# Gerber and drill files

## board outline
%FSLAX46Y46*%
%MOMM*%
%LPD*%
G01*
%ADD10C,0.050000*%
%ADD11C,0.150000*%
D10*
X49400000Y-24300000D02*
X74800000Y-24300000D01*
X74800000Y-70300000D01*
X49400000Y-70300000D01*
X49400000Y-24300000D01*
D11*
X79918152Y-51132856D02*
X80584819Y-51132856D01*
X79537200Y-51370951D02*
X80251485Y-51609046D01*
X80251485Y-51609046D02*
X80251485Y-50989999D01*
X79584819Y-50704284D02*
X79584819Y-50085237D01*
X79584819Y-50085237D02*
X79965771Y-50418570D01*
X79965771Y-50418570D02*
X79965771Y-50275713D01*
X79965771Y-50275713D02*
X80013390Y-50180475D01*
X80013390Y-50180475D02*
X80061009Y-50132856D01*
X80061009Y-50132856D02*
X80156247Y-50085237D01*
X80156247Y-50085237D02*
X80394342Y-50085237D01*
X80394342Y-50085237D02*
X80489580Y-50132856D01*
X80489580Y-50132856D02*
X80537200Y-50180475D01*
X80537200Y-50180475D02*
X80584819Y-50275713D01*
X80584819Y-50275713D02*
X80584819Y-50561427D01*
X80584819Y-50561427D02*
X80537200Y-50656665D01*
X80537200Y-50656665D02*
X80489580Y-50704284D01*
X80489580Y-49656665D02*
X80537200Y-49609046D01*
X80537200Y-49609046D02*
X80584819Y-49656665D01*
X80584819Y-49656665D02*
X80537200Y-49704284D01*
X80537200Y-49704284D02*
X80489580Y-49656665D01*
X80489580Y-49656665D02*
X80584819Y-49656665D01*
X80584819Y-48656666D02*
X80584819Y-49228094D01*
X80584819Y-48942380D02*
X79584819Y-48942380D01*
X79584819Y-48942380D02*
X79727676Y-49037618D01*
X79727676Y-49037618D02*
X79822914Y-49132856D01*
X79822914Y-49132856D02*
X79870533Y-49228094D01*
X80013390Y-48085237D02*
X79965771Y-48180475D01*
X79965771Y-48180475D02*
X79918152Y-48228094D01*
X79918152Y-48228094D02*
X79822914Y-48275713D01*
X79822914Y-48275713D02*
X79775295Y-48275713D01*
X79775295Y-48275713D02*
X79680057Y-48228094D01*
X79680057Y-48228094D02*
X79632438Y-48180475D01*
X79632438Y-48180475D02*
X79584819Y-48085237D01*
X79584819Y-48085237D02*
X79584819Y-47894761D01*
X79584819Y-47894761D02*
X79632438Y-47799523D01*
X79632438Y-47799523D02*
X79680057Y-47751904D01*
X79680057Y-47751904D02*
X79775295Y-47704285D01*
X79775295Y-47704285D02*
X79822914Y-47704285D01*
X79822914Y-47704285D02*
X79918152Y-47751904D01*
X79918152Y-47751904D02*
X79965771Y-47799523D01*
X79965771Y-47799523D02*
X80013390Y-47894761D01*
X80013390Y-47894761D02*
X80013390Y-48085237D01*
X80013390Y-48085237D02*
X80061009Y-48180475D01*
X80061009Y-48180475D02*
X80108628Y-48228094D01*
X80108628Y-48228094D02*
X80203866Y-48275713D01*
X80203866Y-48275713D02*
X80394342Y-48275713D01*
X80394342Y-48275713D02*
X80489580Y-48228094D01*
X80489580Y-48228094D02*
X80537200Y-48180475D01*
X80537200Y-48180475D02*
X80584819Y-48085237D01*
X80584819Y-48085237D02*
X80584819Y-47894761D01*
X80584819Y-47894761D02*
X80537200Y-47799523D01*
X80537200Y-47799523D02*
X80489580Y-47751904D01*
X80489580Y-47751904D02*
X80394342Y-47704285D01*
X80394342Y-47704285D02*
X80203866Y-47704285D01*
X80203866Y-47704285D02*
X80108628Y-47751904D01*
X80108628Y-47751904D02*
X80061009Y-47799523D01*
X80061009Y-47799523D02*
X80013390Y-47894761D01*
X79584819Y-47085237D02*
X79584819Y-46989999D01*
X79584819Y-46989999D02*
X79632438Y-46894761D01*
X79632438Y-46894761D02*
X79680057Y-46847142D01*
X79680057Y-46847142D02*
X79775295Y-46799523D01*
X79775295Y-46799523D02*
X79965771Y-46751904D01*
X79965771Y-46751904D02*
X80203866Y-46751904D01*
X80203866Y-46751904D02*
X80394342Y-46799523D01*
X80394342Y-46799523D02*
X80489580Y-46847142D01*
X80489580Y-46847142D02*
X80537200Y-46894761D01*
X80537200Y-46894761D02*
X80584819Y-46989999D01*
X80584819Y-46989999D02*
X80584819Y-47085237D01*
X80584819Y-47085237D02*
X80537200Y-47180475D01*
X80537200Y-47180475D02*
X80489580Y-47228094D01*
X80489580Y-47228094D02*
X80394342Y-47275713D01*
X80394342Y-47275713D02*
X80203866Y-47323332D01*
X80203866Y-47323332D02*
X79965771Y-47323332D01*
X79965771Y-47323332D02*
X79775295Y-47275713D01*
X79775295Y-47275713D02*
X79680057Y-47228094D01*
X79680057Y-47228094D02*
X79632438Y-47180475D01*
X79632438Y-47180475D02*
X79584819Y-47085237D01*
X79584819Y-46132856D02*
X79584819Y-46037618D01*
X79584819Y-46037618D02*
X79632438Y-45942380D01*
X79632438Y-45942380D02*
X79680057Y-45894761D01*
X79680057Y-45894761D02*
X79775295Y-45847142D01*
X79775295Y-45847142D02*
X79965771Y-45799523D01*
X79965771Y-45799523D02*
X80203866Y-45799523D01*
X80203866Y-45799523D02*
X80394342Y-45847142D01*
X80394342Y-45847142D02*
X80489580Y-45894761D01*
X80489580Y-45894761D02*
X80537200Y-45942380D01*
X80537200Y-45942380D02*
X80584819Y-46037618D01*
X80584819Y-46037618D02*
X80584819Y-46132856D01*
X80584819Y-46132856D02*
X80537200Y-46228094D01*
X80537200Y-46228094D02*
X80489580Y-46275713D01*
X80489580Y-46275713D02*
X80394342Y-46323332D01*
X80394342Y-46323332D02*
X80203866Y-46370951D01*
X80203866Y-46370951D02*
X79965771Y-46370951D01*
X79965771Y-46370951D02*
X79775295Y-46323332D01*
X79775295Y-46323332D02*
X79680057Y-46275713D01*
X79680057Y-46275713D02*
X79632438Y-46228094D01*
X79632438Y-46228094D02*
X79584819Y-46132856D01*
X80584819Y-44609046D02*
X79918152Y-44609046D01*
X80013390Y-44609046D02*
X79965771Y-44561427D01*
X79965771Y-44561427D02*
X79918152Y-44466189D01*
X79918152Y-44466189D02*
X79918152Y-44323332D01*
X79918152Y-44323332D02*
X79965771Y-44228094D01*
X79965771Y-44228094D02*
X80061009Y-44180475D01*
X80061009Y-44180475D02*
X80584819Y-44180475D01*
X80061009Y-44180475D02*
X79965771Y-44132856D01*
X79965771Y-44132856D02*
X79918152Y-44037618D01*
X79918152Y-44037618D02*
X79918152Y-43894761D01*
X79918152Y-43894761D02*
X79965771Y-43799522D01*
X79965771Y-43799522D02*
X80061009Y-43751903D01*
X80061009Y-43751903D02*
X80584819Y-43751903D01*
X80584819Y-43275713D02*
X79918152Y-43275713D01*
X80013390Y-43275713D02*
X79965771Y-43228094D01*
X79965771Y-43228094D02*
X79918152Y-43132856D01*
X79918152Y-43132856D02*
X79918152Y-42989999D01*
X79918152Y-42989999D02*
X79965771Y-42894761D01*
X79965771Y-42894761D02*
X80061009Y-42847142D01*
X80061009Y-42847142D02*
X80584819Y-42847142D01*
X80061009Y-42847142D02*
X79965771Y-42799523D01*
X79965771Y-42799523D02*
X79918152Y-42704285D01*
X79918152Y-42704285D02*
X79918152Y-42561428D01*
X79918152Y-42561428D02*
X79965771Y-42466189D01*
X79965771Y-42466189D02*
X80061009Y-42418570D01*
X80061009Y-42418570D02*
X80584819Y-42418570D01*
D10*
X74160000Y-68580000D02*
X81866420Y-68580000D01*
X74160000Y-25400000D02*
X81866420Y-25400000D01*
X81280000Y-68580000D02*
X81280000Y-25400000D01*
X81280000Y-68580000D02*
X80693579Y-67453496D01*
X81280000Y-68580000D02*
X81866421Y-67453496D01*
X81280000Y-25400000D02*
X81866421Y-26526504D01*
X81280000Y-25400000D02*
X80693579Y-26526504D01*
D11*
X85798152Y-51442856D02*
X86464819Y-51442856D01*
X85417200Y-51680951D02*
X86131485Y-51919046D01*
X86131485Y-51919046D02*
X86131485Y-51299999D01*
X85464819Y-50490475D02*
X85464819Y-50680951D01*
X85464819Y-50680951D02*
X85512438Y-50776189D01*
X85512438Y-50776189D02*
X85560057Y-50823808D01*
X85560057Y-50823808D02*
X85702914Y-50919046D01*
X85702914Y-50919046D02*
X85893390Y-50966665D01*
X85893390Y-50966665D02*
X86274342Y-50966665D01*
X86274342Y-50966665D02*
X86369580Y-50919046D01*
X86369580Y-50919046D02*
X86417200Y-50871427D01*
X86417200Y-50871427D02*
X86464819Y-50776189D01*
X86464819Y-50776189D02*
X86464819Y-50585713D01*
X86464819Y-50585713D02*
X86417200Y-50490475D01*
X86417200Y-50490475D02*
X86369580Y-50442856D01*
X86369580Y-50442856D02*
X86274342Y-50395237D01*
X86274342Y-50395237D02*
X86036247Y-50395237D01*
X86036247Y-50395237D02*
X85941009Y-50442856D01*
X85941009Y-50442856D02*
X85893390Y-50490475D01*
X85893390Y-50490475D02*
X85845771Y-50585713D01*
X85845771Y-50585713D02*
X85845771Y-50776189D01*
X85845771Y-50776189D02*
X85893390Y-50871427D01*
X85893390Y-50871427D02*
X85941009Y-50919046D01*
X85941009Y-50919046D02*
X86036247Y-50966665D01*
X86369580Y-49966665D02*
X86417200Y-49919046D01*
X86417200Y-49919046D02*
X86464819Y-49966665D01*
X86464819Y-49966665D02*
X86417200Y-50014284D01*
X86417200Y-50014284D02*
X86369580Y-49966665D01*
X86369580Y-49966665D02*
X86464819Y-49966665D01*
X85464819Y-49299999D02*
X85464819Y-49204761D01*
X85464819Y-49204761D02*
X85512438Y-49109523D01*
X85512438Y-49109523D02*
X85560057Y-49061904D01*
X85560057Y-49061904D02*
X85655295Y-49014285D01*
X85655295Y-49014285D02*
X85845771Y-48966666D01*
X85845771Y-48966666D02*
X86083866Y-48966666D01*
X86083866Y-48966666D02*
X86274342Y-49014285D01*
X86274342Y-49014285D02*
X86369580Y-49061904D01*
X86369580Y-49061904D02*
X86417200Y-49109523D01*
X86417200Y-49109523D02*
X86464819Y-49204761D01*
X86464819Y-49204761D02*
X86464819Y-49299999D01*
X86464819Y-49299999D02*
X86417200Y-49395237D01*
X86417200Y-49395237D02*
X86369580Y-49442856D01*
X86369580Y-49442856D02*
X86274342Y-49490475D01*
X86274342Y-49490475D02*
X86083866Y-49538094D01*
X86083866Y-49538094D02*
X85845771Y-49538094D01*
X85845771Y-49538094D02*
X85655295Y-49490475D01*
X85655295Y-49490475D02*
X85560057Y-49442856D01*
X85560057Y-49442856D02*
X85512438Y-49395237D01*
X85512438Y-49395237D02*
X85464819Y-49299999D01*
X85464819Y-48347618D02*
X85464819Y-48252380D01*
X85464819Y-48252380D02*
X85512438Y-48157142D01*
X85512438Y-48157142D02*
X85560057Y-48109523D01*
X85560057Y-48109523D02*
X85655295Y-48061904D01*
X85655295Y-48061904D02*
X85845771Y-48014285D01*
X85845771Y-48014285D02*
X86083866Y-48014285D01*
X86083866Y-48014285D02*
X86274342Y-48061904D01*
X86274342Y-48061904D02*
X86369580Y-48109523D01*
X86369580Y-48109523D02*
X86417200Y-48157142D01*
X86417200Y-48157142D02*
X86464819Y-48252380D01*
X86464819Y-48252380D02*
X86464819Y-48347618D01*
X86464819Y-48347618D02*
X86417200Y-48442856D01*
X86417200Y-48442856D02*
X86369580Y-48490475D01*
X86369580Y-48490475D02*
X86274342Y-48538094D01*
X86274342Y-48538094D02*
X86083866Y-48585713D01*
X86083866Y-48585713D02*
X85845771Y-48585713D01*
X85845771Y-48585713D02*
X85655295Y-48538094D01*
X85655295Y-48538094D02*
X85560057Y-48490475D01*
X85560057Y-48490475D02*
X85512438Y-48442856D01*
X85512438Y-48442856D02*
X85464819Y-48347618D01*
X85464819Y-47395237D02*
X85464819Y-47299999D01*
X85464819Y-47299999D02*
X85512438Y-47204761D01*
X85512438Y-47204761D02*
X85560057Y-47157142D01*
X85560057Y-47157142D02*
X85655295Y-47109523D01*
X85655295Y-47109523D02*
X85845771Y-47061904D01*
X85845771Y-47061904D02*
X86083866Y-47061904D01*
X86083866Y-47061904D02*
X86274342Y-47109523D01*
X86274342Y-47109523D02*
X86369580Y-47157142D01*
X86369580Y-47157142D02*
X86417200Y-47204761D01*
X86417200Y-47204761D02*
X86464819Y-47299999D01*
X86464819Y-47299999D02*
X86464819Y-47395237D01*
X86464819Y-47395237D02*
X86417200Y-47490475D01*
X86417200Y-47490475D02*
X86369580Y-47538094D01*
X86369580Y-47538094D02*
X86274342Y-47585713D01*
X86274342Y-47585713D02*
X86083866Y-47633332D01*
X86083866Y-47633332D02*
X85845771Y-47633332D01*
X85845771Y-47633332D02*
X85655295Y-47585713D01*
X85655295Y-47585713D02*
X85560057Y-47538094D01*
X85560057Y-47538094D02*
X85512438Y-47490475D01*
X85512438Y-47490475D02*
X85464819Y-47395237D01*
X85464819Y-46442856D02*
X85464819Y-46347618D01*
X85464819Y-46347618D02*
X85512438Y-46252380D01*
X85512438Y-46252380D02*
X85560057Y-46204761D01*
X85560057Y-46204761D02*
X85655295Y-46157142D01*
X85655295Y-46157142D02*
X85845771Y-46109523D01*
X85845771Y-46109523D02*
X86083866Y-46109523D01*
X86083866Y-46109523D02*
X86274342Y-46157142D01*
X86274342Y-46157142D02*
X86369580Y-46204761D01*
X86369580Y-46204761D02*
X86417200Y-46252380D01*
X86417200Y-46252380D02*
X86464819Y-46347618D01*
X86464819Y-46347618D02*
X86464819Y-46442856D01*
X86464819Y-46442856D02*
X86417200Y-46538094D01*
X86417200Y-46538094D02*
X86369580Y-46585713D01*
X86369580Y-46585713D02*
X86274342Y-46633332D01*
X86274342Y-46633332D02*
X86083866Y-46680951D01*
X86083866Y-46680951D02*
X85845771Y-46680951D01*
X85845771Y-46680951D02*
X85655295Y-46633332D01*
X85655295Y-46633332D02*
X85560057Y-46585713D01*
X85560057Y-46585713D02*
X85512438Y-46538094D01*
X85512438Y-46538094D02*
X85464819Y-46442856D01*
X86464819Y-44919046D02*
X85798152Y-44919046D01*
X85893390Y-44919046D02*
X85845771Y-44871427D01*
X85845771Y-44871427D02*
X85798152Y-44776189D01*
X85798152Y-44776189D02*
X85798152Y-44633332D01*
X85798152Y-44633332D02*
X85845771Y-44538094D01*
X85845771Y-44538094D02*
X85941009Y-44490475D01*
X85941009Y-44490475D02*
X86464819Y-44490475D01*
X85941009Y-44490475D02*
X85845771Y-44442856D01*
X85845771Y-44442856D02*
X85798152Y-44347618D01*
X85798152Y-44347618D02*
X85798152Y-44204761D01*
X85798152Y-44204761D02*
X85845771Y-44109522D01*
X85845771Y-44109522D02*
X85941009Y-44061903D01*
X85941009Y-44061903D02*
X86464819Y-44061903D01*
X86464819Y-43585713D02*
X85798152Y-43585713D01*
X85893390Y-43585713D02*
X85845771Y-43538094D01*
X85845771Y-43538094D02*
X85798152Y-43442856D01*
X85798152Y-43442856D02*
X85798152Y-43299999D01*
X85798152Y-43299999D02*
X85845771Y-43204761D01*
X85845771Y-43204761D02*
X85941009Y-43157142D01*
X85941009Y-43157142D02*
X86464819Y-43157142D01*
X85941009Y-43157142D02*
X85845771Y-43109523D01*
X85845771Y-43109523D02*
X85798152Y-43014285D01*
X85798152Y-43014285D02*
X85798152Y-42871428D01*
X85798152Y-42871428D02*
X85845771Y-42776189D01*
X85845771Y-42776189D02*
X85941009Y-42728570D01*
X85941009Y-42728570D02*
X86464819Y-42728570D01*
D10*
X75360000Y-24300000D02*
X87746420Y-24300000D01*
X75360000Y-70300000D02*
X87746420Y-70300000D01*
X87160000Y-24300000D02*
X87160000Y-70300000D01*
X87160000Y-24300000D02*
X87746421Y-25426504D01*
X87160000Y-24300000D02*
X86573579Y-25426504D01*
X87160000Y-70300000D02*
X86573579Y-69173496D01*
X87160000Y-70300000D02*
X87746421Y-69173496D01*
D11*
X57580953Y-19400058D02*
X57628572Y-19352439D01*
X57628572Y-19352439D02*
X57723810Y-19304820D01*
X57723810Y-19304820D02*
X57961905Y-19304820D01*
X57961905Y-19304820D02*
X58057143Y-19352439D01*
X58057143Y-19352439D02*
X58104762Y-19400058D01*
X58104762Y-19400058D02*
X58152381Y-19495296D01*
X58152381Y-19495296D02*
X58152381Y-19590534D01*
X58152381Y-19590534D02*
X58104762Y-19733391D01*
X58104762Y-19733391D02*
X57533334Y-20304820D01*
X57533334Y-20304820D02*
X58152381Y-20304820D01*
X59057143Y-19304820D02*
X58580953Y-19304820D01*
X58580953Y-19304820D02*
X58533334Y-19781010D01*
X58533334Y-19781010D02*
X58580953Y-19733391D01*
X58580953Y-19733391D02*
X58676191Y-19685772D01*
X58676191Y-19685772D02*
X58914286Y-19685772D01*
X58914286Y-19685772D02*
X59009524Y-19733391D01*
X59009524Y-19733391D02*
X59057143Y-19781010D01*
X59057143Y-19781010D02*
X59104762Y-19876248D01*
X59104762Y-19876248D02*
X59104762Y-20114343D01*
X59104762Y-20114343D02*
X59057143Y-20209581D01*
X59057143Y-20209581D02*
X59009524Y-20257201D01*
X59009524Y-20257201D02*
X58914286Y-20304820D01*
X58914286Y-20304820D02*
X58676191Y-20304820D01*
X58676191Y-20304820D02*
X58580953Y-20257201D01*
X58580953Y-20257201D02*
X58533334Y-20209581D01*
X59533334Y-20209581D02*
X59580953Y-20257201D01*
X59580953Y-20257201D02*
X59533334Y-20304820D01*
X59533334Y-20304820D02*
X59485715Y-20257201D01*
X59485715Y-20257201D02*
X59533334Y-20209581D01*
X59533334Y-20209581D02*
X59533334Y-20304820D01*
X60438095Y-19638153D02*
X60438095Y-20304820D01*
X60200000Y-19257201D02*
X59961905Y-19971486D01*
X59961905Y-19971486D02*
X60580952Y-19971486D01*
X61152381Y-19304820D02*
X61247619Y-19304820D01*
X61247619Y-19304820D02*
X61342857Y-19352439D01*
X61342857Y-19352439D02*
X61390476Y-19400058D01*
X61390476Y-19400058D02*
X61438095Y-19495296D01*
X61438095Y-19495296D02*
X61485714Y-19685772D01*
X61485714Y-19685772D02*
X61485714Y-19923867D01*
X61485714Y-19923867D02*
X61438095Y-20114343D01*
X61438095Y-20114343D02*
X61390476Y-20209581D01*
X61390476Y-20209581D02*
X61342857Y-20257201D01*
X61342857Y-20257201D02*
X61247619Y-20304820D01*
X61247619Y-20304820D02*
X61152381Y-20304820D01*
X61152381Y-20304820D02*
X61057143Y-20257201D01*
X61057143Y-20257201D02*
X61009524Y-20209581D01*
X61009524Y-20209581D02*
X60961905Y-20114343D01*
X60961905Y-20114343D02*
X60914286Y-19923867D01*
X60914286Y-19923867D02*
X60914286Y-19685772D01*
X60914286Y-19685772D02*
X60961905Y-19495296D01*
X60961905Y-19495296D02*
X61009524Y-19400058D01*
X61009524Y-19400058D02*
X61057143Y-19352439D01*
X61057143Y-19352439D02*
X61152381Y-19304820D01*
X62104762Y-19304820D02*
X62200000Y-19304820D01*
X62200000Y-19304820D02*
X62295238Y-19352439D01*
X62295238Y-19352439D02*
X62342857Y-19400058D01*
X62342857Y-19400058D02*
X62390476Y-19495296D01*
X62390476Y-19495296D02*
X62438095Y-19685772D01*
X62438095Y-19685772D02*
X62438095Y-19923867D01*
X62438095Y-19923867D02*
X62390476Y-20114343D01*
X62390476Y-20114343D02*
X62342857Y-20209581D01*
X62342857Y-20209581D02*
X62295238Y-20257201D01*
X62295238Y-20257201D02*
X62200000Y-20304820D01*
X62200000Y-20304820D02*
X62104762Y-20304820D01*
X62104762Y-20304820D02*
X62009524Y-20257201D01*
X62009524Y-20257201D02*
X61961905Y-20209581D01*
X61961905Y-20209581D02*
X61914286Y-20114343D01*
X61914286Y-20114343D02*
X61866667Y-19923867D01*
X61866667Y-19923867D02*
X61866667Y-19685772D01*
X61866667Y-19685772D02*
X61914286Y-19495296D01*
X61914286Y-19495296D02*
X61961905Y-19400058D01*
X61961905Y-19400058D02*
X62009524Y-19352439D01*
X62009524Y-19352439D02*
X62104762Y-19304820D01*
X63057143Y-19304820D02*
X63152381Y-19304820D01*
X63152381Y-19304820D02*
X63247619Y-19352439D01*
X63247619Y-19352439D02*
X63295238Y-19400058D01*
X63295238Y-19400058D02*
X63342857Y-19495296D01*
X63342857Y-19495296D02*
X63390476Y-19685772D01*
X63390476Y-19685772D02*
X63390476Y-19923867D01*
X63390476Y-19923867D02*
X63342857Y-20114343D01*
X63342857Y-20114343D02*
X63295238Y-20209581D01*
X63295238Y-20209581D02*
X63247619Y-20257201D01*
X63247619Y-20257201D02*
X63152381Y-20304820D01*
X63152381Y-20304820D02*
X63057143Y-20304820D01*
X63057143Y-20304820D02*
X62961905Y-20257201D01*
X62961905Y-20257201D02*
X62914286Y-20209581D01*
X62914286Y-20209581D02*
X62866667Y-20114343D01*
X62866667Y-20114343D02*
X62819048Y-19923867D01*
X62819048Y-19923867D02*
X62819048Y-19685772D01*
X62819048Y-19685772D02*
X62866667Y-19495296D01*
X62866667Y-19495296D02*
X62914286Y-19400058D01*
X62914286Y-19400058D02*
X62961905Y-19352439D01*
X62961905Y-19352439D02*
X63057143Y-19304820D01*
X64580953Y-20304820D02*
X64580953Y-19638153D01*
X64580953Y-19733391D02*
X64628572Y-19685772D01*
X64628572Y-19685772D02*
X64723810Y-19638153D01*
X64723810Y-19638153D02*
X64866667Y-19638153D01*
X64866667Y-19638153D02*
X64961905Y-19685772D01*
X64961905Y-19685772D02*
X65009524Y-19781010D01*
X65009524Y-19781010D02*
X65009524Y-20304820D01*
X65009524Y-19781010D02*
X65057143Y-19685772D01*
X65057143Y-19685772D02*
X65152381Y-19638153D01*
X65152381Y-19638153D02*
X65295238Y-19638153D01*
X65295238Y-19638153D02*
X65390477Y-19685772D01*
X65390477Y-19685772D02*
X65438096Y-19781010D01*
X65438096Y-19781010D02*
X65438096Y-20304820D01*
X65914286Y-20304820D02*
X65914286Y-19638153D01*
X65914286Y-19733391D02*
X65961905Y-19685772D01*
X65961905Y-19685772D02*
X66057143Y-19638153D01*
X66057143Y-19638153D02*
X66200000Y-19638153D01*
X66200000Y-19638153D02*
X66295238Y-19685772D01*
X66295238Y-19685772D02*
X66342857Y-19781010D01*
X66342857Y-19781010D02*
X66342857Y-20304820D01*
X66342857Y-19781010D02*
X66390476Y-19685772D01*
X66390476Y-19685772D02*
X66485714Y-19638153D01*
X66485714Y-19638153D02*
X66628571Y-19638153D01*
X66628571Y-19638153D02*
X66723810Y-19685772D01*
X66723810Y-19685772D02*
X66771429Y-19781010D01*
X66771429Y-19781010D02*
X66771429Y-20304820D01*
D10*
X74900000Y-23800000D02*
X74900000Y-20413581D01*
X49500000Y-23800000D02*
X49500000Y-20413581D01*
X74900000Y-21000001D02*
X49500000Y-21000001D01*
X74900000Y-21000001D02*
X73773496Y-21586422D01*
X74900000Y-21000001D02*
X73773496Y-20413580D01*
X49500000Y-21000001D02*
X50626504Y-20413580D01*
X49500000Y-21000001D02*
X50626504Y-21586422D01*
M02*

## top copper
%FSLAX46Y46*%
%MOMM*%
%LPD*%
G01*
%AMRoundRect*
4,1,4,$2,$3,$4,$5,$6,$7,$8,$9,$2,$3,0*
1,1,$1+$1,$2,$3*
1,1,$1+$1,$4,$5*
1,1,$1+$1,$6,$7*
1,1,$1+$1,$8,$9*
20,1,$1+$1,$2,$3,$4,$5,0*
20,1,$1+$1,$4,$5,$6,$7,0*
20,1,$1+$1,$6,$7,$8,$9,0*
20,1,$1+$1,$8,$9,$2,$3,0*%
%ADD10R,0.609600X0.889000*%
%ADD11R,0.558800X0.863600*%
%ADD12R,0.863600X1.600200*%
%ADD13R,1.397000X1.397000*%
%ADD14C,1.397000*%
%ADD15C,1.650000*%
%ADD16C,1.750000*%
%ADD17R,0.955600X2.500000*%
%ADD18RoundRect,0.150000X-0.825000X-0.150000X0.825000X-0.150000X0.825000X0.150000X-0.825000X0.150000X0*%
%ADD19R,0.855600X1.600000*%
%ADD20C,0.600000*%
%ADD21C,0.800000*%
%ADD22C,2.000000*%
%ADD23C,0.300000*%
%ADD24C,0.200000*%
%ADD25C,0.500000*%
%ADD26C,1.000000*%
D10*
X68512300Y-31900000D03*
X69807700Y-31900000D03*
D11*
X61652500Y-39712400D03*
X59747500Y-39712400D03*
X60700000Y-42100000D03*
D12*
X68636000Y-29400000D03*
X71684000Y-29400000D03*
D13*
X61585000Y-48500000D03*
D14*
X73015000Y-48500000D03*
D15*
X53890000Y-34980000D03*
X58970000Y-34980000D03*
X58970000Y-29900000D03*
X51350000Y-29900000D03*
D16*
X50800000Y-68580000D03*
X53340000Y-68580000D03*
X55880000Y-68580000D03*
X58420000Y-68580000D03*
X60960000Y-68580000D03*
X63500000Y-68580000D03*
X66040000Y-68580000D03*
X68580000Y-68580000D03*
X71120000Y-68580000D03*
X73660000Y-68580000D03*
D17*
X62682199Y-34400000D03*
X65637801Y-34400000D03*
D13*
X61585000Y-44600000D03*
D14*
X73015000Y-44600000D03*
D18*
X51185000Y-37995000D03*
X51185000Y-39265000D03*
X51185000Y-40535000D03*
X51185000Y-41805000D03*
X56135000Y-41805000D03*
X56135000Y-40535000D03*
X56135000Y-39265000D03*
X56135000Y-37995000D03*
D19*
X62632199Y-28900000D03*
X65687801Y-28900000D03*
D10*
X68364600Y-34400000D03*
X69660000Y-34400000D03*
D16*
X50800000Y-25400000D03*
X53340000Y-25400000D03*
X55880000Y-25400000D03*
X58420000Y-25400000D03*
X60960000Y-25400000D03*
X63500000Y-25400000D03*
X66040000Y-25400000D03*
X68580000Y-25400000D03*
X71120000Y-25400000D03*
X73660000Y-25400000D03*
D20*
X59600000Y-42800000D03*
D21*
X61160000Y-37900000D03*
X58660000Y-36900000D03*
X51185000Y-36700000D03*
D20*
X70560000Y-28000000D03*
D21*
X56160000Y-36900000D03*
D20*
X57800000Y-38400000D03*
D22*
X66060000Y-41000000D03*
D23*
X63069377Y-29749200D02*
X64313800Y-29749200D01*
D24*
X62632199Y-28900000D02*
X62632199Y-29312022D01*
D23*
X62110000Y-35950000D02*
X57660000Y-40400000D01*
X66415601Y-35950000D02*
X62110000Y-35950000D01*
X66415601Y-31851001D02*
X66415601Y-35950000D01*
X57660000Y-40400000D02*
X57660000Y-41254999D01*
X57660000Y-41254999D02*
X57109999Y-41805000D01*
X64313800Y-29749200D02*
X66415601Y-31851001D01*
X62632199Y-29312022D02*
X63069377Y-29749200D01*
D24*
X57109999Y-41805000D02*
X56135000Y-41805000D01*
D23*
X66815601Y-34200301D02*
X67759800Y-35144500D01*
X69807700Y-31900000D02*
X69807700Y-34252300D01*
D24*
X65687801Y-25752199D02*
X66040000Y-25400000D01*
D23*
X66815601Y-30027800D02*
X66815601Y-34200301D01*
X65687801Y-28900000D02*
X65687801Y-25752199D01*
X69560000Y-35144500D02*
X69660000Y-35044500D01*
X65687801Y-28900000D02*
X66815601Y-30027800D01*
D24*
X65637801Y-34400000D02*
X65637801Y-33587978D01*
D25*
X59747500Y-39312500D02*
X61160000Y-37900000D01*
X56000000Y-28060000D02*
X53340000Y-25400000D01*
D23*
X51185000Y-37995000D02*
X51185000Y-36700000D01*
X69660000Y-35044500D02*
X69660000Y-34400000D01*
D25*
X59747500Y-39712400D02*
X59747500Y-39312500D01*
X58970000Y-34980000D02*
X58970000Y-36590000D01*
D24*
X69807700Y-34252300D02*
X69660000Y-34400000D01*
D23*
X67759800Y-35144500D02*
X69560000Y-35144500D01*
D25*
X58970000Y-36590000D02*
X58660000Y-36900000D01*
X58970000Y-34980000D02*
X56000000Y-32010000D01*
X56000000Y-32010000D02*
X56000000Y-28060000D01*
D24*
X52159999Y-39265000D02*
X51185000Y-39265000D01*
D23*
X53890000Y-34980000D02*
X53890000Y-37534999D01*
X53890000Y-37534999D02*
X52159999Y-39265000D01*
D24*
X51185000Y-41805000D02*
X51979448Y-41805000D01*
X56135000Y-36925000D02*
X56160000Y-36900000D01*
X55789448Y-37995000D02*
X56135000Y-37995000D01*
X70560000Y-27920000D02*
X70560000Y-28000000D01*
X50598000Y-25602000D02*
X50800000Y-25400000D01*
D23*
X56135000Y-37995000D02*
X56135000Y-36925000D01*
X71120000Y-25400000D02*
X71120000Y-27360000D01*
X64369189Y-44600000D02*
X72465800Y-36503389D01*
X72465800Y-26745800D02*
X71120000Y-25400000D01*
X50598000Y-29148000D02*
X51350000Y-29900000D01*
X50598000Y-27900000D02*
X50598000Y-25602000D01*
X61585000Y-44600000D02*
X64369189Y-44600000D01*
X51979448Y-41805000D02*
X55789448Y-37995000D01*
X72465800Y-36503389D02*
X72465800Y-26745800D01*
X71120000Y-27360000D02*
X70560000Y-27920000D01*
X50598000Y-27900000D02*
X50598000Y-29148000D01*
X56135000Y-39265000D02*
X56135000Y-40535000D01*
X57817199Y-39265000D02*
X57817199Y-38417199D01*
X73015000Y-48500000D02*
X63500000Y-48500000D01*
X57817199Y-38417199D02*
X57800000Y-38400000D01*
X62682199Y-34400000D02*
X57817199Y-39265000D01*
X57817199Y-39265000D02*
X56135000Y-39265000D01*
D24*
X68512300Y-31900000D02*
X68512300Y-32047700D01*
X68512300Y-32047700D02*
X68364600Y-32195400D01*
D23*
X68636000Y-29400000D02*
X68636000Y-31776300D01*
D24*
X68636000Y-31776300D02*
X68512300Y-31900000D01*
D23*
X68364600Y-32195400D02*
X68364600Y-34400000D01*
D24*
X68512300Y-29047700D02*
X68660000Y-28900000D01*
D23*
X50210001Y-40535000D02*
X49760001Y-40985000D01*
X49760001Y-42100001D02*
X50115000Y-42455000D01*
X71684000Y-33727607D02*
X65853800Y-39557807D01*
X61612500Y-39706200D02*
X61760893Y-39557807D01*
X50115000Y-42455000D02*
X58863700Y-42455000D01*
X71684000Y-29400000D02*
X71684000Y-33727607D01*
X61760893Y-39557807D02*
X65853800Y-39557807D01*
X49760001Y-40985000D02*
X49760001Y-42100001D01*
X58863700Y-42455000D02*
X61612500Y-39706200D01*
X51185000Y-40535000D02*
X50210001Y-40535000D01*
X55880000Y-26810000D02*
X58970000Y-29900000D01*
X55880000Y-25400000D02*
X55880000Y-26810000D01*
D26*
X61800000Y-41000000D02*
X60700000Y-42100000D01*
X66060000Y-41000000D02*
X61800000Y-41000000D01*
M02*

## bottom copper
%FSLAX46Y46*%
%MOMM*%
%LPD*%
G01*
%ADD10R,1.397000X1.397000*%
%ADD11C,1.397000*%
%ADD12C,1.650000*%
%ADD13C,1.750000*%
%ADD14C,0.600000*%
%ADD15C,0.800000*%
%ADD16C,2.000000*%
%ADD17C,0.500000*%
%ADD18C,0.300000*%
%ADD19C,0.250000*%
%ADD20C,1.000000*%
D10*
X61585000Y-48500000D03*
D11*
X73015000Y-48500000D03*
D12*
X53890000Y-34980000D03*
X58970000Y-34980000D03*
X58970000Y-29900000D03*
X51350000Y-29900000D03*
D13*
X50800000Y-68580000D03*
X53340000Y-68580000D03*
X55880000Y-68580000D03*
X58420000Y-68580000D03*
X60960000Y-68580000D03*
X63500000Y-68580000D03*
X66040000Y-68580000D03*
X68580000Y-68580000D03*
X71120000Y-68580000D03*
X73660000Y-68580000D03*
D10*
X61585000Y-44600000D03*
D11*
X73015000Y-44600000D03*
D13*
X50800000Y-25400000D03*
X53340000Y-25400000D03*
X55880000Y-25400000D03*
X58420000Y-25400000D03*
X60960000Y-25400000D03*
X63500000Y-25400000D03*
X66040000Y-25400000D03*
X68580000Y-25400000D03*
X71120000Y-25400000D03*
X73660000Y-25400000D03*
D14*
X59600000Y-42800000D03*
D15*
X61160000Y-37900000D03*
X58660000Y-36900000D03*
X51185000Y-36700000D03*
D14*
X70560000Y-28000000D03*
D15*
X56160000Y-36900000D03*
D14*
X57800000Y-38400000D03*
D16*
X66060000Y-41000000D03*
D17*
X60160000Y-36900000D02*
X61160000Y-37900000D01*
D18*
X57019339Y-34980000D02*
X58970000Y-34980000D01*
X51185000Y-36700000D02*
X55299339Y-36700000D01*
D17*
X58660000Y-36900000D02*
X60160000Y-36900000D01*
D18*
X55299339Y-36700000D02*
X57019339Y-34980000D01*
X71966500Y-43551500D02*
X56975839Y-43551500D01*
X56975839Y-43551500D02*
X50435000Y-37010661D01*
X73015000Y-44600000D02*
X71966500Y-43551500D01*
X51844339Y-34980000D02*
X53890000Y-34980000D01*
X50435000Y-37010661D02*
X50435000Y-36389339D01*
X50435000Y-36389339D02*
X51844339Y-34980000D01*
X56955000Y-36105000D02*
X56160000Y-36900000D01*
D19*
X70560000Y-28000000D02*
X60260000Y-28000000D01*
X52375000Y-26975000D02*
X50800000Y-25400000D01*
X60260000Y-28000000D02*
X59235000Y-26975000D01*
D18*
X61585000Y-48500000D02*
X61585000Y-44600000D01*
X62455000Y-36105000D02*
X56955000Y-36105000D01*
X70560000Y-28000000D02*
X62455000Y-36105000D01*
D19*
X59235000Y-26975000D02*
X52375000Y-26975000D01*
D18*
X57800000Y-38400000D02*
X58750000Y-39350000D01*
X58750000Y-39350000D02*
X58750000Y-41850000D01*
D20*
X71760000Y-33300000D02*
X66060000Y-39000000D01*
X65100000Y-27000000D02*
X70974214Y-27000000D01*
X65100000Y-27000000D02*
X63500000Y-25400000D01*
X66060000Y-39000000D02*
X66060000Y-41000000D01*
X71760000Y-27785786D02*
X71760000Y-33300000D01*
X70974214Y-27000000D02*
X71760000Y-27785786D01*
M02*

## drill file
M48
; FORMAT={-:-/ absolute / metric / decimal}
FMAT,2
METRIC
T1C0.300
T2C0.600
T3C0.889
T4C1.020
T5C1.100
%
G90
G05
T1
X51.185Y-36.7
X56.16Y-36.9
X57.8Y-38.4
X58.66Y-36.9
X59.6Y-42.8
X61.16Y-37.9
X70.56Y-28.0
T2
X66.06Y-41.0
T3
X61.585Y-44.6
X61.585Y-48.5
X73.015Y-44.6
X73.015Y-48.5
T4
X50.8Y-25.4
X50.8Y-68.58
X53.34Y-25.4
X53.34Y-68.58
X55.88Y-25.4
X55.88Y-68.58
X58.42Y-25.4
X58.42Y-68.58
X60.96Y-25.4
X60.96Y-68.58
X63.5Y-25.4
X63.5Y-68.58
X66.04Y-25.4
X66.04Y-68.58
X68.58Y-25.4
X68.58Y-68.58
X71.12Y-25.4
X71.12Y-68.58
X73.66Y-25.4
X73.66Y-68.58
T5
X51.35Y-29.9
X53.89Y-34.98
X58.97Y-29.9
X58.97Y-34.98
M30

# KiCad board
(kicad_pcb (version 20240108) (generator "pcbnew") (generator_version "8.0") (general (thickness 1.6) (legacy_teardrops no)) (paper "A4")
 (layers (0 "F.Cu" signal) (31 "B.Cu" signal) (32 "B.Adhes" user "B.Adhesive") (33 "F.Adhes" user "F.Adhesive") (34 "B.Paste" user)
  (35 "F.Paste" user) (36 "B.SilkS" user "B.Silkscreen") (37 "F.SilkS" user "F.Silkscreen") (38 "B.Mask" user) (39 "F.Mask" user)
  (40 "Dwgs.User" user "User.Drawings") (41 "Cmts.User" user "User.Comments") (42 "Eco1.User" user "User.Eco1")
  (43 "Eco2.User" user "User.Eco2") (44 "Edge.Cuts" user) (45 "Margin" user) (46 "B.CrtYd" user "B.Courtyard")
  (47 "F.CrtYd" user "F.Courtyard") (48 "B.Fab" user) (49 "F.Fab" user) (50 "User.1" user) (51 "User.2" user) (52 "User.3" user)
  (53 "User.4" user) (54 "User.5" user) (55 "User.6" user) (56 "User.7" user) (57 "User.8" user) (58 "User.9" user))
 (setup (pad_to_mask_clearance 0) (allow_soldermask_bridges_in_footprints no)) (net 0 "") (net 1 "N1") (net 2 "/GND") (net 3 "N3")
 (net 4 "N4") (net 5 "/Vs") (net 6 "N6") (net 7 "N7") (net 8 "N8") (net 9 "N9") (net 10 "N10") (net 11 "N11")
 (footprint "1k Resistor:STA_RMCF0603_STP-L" (layer "F.Cu") (at 69.16 31.9)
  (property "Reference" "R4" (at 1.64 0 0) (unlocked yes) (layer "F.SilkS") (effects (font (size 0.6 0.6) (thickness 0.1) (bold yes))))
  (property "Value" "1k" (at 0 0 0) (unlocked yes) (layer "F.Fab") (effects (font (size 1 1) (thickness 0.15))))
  (pad "1" smd rect (at -0.6477 0) (size 0.6096 0.889) (layers "F.Cu" "F.Paste" "F.Mask") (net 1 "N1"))
  (pad "2" smd rect (at 0.6477 0) (size 0.6096 0.889) (layers "F.Cu" "F.Paste" "F.Mask") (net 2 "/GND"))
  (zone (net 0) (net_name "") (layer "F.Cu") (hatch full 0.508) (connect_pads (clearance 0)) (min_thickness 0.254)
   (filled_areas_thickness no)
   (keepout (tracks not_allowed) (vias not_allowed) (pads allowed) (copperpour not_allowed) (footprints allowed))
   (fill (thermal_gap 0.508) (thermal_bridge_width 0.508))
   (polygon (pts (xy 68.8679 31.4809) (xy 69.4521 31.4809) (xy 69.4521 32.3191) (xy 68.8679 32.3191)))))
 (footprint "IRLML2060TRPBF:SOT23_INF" (layer "F.Cu") (at 60.7 40.9062 180)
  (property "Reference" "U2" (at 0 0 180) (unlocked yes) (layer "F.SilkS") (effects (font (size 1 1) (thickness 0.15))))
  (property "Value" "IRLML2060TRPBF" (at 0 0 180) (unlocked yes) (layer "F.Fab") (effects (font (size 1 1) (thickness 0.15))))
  (pad "1" smd rect (at -0.9525 1.1938 180) (size 0.5588 0.8636) (layers "F.Cu" "F.Paste" "F.Mask") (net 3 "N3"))
  (pad "2" smd rect (at 0.9525 1.1938 180) (size 0.5588 0.8636) (layers "F.Cu" "F.Paste" "F.Mask") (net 2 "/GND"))
  (pad "3" smd rect (at 0 -1.1938 180) (size 0.5588 0.8636) (layers "F.Cu" "F.Paste" "F.Mask") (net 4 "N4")))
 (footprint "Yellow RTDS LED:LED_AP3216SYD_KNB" (layer "F.Cu") (at 70.16 29.4)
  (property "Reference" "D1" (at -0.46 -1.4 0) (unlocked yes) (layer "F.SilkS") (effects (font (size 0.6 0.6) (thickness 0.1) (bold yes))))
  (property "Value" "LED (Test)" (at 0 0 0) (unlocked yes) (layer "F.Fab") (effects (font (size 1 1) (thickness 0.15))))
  (pad "1" smd rect (at -1.524 0) (size 0.8636 1.6002) (layers "F.Cu" "F.Paste" "F.Mask") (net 1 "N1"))
  (pad "2" smd rect (at 1.524 0) (size 0.8636 1.6002) (layers "F.Cu" "F.Paste" "F.Mask") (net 3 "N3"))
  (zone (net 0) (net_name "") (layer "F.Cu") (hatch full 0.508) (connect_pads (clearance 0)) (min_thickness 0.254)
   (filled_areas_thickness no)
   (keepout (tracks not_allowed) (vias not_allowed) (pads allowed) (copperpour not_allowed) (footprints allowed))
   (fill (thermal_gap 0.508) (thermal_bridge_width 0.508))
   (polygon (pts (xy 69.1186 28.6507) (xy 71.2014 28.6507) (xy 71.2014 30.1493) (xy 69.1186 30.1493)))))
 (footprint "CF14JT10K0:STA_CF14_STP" (layer "F.Cu") (at 61.585 48.5)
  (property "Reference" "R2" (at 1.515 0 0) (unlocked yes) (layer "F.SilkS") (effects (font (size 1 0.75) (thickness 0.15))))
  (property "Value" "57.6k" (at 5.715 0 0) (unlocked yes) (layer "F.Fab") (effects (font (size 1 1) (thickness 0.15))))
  (pad "1" thru_hole rect (at 0 0) (size 1.397 1.397) (drill 0.889) (layers "*.Cu" "*.Mask") (remove_unused_layers no) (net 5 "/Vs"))
  (pad "2" thru_hole circle (at 11.43 0) (size 1.397 1.397) (drill 0.889) (layers "*.Cu" "*.Mask") (remove_unused_layers no) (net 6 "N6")))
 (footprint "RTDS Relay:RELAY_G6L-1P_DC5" (layer "F.Cu") (at 55.16 32.44)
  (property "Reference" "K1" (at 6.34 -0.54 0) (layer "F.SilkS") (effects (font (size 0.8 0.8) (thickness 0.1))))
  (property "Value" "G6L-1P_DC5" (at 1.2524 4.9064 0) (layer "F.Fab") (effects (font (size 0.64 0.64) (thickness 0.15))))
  (pad "2" thru_hole circle (at -1.27 2.54) (size 1.65 1.65) (drill 1.1) (layers "*.Cu" "*.Mask") (remove_unused_layers no) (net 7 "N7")
   (solder_mask_margin 0.102))
  (pad "4" thru_hole circle (at 3.81 2.54) (size 1.65 1.65) (drill 1.1) (layers "*.Cu" "*.Mask") (remove_unused_layers no) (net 2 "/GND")
   (solder_mask_margin 0.102))
  (pad "5" thru_hole circle (at 3.81 -2.54) (size 1.65 1.65) (drill 1.1) (layers "*.Cu" "*.Mask") (remove_unused_layers no) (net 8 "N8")
   (solder_mask_margin 0.102))
  (pad "8" thru_hole circle (at -3.81 -2.54) (size 1.65 1.65) (drill 1.1) (layers "*.Cu" "*.Mask") (remove_unused_layers no) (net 5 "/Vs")
   (solder_mask_margin 0.102)))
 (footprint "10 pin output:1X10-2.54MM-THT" (layer "F.Cu") (at 50.8 68.58)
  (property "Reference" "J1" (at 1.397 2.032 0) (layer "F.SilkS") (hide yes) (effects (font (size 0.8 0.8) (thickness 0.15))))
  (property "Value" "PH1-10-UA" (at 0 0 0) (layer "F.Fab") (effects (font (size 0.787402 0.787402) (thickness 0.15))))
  (pad "1" thru_hole circle (at 0 0) (size 1.75 1.75) (drill 1.02) (layers "*.Cu" "*.Mask") (remove_unused_layers no)
   (solder_mask_margin 0.102))
  (pad "2" thru_hole circle (at 2.54 0) (size 1.75 1.75) (drill 1.02) (layers "*.Cu" "*.Mask") (remove_unused_layers no)
   (solder_mask_margin 0.102))
  (pad "3" thru_hole circle (at 5.08 0) (size 1.75 1.75) (drill 1.02) (layers "*.Cu" "*.Mask") (remove_unused_layers no)
   (solder_mask_margin 0.102))
  (pad "4" thru_hole circle (at 7.62 0) (size 1.75 1.75) (drill 1.02) (layers "*.Cu" "*.Mask") (remove_unused_layers no)
   (solder_mask_margin 0.102))
  (pad "5" thru_hole circle (at 10.16 0) (size 1.75 1.75) (drill 1.02) (layers "*.Cu" "*.Mask") (remove_unused_layers no)
   (solder_mask_margin 0.102))
  (pad "6" thru_hole circle (at 12.7 0) (size 1.75 1.75) (drill 1.02) (layers "*.Cu" "*.Mask") (remove_unused_layers no)
   (solder_mask_margin 0.102))
  (pad "7" thru_hole circle (at 15.24 0) (size 1.75 1.75) (drill 1.02) (layers "*.Cu" "*.Mask") (remove_unused_layers no)
   (solder_mask_margin 0.102))
  (pad "8" thru_hole circle (at 17.78 0) (size 1.75 1.75) (drill 1.02) (layers "*.Cu" "*.Mask") (remove_unused_layers no)
   (solder_mask_margin 0.102))
  (pad "9" thru_hole circle (at 20.32 0) (size 1.75 1.75) (drill 1.02) (layers "*.Cu" "*.Mask") (remove_unused_layers no)
   (solder_mask_margin 0.102))
  (pad "10" thru_hole circle (at 22.86 0) (size 1.75 1.75) (drill 1.02) (layers "*.Cu" "*.Mask") (remove_unused_layers no)
   (solder_mask_margin 0.102)))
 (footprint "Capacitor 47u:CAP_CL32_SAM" (layer "F.Cu") (at 64.16 34.4)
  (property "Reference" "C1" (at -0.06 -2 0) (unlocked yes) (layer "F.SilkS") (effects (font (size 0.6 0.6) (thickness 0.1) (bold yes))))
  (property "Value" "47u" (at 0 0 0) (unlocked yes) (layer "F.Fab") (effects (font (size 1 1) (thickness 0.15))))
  (pad "1" smd rect (at -1.477801 0) (size 0.9556 2.5) (layers "F.Cu" "F.Paste" "F.Mask") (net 6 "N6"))
  (pad "2" smd rect (at 1.477801 0) (size 0.9556 2.5) (layers "F.Cu" "F.Paste" "F.Mask") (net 2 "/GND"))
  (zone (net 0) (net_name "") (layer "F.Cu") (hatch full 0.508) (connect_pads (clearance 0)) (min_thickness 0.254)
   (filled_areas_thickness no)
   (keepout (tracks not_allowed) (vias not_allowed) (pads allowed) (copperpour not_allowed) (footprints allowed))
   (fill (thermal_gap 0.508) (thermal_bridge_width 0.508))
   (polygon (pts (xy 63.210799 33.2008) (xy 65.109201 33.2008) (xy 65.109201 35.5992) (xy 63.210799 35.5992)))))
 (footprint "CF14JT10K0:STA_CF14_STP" (layer "F.Cu") (at 61.585 44.6)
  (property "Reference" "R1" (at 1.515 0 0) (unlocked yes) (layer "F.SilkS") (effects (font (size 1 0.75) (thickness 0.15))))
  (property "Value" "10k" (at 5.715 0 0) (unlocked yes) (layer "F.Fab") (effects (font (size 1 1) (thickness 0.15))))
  (pad "1" thru_hole rect (at 0 0) (size 1.397 1.397) (drill 0.889) (layers "*.Cu" "*.Mask") (remove_unused_layers no) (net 5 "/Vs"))
  (pad "2" thru_hole circle (at 11.43 0) (size 1.397 1.397) (drill 0.889) (layers "*.Cu" "*.Mask") (remove_unused_layers no) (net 7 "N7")))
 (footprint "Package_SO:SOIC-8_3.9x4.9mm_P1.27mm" (layer "F.Cu") (at 53.66 39.9)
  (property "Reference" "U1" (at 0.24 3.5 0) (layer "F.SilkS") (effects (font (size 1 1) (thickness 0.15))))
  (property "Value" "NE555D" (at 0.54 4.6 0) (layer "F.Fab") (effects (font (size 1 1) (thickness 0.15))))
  (pad "1" smd roundrect (at -2.475 -1.905) (size 1.95 0.6) (layers "F.Cu" "F.Paste" "F.Mask") (roundrect_rratio 0.25) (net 2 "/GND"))
  (pad "2" smd roundrect (at -2.475 -0.635) (size 1.95 0.6) (layers "F.Cu" "F.Paste" "F.Mask") (roundrect_rratio 0.25) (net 7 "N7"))
  (pad "3" smd roundrect (at -2.475 0.635) (size 1.95 0.6) (layers "F.Cu" "F.Paste" "F.Mask") (roundrect_rratio 0.25) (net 3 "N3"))
  (pad "4" smd roundrect (at -2.475 1.905) (size 1.95 0.6) (layers "F.Cu" "F.Paste" "F.Mask") (roundrect_rratio 0.25) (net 5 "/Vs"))
  (pad "5" smd roundrect (at 2.475 1.905) (size 1.95 0.6) (layers "F.Cu" "F.Paste" "F.Mask") (roundrect_rratio 0.25) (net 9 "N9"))
  (pad "6" smd roundrect (at 2.475 0.635) (size 1.95 0.6) (layers "F.Cu" "F.Paste" "F.Mask") (roundrect_rratio 0.25) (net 6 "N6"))
  (pad "7" smd roundrect (at 2.475 -0.635) (size 1.95 0.6) (layers "F.Cu" "F.Paste" "F.Mask") (roundrect_rratio 0.25) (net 6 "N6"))
  (pad "8" smd roundrect (at 2.475 -1.905) (size 1.95 0.6) (layers "F.Cu" "F.Paste" "F.Mask") (roundrect_rratio 0.25) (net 5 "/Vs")))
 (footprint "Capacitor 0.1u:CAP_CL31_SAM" (layer "F.Cu") (at 64.16 28.9)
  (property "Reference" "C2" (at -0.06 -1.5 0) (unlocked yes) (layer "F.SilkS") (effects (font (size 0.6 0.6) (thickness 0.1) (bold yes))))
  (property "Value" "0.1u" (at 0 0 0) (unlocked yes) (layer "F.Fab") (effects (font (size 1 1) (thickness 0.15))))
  (pad "1" smd rect (at -1.527801 0) (size 0.8556 1.6) (layers "F.Cu" "F.Paste" "F.Mask") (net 9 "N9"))
  (pad "2" smd rect (at 1.527801 0) (size 0.8556 1.6) (layers "F.Cu" "F.Paste" "F.Mask") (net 2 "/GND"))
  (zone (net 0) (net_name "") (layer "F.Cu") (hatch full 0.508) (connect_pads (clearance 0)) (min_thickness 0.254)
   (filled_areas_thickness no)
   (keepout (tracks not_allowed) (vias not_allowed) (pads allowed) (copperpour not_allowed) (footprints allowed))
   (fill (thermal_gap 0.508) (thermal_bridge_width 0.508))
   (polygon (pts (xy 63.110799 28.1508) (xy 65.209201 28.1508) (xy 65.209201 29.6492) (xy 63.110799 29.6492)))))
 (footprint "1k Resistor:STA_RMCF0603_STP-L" (layer "F.Cu") (at 69.0123 34.4)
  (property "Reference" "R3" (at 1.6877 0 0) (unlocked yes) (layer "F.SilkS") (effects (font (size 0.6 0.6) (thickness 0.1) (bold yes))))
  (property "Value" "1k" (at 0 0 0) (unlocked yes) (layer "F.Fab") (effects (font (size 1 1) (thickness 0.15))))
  (pad "1" smd rect (at -0.6477 0) (size 0.6096 0.889) (layers "F.Cu" "F.Paste" "F.Mask") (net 1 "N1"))
  (pad "2" smd rect (at 0.6477 0) (size 0.6096 0.889) (layers "F.Cu" "F.Paste" "F.Mask") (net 2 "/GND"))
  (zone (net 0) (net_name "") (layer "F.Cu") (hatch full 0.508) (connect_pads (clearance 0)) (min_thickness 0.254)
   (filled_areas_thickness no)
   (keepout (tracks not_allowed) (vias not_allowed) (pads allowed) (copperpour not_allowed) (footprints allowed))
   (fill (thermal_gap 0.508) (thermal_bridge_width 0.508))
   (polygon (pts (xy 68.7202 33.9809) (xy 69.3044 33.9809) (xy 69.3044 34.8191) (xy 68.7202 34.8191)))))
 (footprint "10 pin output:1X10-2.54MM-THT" (layer "F.Cu") (at 50.8 25.4)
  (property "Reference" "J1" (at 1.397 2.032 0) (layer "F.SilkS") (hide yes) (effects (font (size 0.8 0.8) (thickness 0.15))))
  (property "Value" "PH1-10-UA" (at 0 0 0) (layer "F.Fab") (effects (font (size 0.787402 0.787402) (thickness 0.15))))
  (pad "1" thru_hole circle (at 0 0) (size 1.75 1.75) (drill 1.02) (layers "*.Cu" "*.Mask") (remove_unused_layers no) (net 5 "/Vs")
   (solder_mask_margin 0.102))
  (pad "2" thru_hole circle (at 2.54 0) (size 1.75 1.75) (drill 1.02) (layers "*.Cu" "*.Mask") (remove_unused_layers no) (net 2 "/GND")
   (solder_mask_margin 0.102))
  (pad "3" thru_hole circle (at 5.08 0) (size 1.75 1.75) (drill 1.02) (layers "*.Cu" "*.Mask") (remove_unused_layers no) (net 8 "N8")
   (solder_mask_margin 0.102))
  (pad "4" thru_hole circle (at 7.62 0) (size 1.75 1.75) (drill 1.02) (layers "*.Cu" "*.Mask") (remove_unused_layers no) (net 2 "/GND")
   (solder_mask_margin 0.102))
  (pad "5" thru_hole circle (at 10.16 0) (size 1.75 1.75) (drill 1.02) (layers "*.Cu" "*.Mask") (remove_unused_layers no) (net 2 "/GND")
   (solder_mask_margin 0.102))
  (pad "6" thru_hole circle (at 12.7 0) (size 1.75 1.75) (drill 1.02) (layers "*.Cu" "*.Mask") (remove_unused_layers no) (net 4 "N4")
   (solder_mask_margin 0.102))
  (pad "7" thru_hole circle (at 15.24 0) (size 1.75 1.75) (drill 1.02) (layers "*.Cu" "*.Mask") (remove_unused_layers no) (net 2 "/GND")
   (solder_mask_margin 0.102))
  (pad "8" thru_hole circle (at 17.78 0) (size 1.75 1.75) (drill 1.02) (layers "*.Cu" "*.Mask") (remove_unused_layers no) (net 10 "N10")
   (solder_mask_margin 0.102))
  (pad "9" thru_hole circle (at 20.32 0) (size 1.75 1.75) (drill 1.02) (layers "*.Cu" "*.Mask") (remove_unused_layers no) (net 5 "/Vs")
   (solder_mask_margin 0.102))
  (pad "10" thru_hole circle (at 22.86 0) (size 1.75 1.75) (drill 1.02) (layers "*.Cu" "*.Mask") (remove_unused_layers no) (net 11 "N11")
   (solder_mask_margin 0.102)))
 (gr_rect (start 49.4 24.3) (end 74.8 70.3) (stroke (width 0.05) (type default)) (fill none) (layer "Edge.Cuts"))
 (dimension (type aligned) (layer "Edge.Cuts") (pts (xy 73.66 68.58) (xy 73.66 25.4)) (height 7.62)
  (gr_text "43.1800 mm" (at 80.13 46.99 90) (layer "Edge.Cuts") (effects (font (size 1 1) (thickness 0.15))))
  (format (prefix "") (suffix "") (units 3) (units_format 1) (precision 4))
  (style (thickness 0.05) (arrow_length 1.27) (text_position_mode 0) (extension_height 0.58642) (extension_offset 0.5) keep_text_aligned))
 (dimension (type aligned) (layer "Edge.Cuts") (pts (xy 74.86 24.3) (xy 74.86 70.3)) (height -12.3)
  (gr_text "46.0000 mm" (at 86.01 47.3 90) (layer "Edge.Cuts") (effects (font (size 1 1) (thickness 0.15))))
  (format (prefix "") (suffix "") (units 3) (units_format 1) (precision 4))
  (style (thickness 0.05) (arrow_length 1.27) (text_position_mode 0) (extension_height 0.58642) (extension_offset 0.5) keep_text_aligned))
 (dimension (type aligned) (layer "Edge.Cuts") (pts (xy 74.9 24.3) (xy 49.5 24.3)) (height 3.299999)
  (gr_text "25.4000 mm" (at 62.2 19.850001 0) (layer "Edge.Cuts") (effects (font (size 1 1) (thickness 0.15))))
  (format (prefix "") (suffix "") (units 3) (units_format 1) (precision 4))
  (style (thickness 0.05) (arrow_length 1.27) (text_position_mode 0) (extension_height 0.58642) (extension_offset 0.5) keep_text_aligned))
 (via (at 59.6 42.8) (size 0.6) (drill 0.3) (layers "F.Cu" "B.Cu") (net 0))
 (segment (start 63.069377 29.7492) (end 64.3138 29.7492) (width 0.3) (layer "F.Cu") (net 9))
 (segment (start 62.632199 28.9) (end 62.632199 29.312022) (width 0.2) (layer "F.Cu") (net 9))
 (segment (start 62.11 35.95) (end 57.66 40.4) (width 0.3) (layer "F.Cu") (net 9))
 (segment (start 66.415601 35.95) (end 62.11 35.95) (width 0.3) (layer "F.Cu") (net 9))
 (segment (start 66.415601 31.851001) (end 66.415601 35.95) (width 0.3) (layer "F.Cu") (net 9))
 (segment (start 57.66 40.4) (end 57.66 41.254999) (width 0.3) (layer "F.Cu") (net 9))
 (segment (start 57.66 41.254999) (end 57.109999 41.805) (width 0.3) (layer "F.Cu") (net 9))
 (segment (start 64.3138 29.7492) (end 66.415601 31.851001) (width 0.3) (layer "F.Cu") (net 9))
 (segment (start 62.632199 29.312022) (end 63.069377 29.7492) (width 0.3) (layer "F.Cu") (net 9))
 (segment (start 57.109999 41.805) (end 56.135 41.805) (width 0.2) (layer "F.Cu") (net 9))
 (segment (start 66.815601 34.200301) (end 67.7598 35.1445) (width 0.3) (layer "F.Cu") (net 2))
 (segment (start 69.8077 31.9) (end 69.8077 34.2523) (width 0.3) (layer "F.Cu") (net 2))
 (segment (start 65.687801 25.752199) (end 66.04 25.4) (width 0.2) (layer "F.Cu") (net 2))
 (segment (start 66.815601 30.0278) (end 66.815601 34.200301) (width 0.3) (layer "F.Cu") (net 2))
 (segment (start 65.687801 28.9) (end 65.687801 25.752199) (width 0.3) (layer "F.Cu") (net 2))
 (segment (start 69.56 35.1445) (end 69.66 35.0445) (width 0.3) (layer "F.Cu") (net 2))
 (segment (start 65.687801 28.9) (end 66.815601 30.0278) (width 0.3) (layer "F.Cu") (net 2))
 (segment (start 65.637801 34.4) (end 65.637801 33.587978) (width 0.2) (layer "F.Cu") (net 2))
 (segment (start 59.7475 39.3125) (end 61.16 37.9) (width 0.5) (layer "F.Cu") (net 2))
 (segment (start 56 28.06) (end 53.34 25.4) (width 0.5) (layer "F.Cu") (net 2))
 (segment (start 51.185 37.995) (end 51.185 36.7) (width 0.3) (layer "F.Cu") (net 2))
 (segment (start 69.66 35.0445) (end 69.66 34.4) (width 0.3) (layer "F.Cu") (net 2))
 (segment (start 59.7475 39.7124) (end 59.7475 39.3125) (width 0.5) (layer "F.Cu") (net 2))
 (segment (start 58.97 34.98) (end 58.97 36.59) (width 0.5) (layer "F.Cu") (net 2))
 (segment (start 69.8077 34.2523) (end 69.66 34.4) (width 0.2) (layer "F.Cu") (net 2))
 (segment (start 67.7598 35.1445) (end 69.56 35.1445) (width 0.3) (layer "F.Cu") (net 2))
 (segment (start 58.97 36.59) (end 58.66 36.9) (width 0.5) (layer "F.Cu") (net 2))
 (segment (start 58.97 34.98) (end 56 32.01) (width 0.5) (layer "F.Cu") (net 2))
 (segment (start 56 32.01) (end 56 28.06) (width 0.5) (layer "F.Cu") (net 2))
 (via (at 61.16 37.9) (size 0.8) (drill 0.3) (layers "F.Cu" "B.Cu") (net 2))
 (via (at 58.66 36.9) (size 0.8) (drill 0.3) (layers "F.Cu" "B.Cu") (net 2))
 (via (at 51.185 36.7) (size 0.8) (drill 0.3) (layers "F.Cu" "B.Cu") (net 2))
 (segment (start 60.16 36.9) (end 61.16 37.9) (width 0.5) (layer "B.Cu") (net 2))
 (segment (start 57.019339 34.98) (end 58.97 34.98) (width 0.3) (layer "B.Cu") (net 2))
 (segment (start 51.185 36.7) (end 55.299339 36.7) (width 0.3) (layer "B.Cu") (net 2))
 (segment (start 58.66 36.9) (end 60.16 36.9) (width 0.5) (layer "B.Cu") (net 2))
 (segment (start 55.299339 36.7) (end 57.019339 34.98) (width 0.3) (layer "B.Cu") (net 2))
 (segment (start 52.159999 39.265) (end 51.185 39.265) (width 0.2) (layer "F.Cu") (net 7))
 (segment (start 53.89 34.98) (end 53.89 37.534999) (width 0.3) (layer "F.Cu") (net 7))
 (segment (start 53.89 37.534999) (end 52.159999 39.265) (width 0.3) (layer "F.Cu") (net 7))
 (segment (start 71.9665 43.5515) (end 56.975839 43.5515) (width 0.3) (layer "B.Cu") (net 7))
 (segment (start 56.975839 43.5515) (end 50.435 37.010661) (width 0.3) (layer "B.Cu") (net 7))
 (segment (start 73.015 44.6) (end 71.9665 43.5515) (width 0.3) (layer "B.Cu") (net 7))
 (segment (start 51.844339 34.98) (end 53.89 34.98) (width 0.3) (layer "B.Cu") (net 7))
 (segment (start 50.435 37.010661) (end 50.435 36.389339) (width 0.3) (layer "B.Cu") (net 7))
 (segment (start 50.435 36.389339) (end 51.844339 34.98) (width 0.3) (layer "B.Cu") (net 7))
 (segment (start 51.185 41.805) (end 51.979448 41.805) (width 0.2) (layer "F.Cu") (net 5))
 (segment (start 56.135 36.925) (end 56.16 36.9) (width 0.2) (layer "F.Cu") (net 5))
 (segment (start 55.789448 37.995) (end 56.135 37.995) (width 0.2) (layer "F.Cu") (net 5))
 (segment (start 70.56 27.92) (end 70.56 28) (width 0.2) (layer "F.Cu") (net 5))
 (segment (start 50.598 25.602) (end 50.8 25.4) (width 0.2) (layer "F.Cu") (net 5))
 (segment (start 56.135 37.995) (end 56.135 36.925) (width 0.3) (layer "F.Cu") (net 5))
 (segment (start 71.12 25.4) (end 71.12 27.36) (width 0.3) (layer "F.Cu") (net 5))
 (segment (start 64.369189 44.6) (end 72.4658 36.503389) (width 0.3) (layer "F.Cu") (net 5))
 (segment (start 72.4658 26.7458) (end 71.12 25.4) (width 0.3) (layer "F.Cu") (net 5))
 (segment (start 50.598 29.148) (end 51.35 29.9) (width 0.3) (layer "F.Cu") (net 5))
 (segment (start 50.598 27.9) (end 50.598 25.602) (width 0.3) (layer "F.Cu") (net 5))
 (segment (start 61.585 44.6) (end 64.369189 44.6) (width 0.3) (layer "F.Cu") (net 5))
 (segment (start 51.979448 41.805) (end 55.789448 37.995) (width 0.3) (layer "F.Cu") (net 5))
 (segment (start 72.4658 36.503389) (end 72.4658 26.7458) (width 0.3) (layer "F.Cu") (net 5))
 (segment (start 71.12 27.36) (end 70.56 27.92) (width 0.3) (layer "F.Cu") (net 5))
 (segment (start 50.598 27.9) (end 50.598 29.148) (width 0.3) (layer "F.Cu") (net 5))
 (via (at 70.56 28) (size 0.6) (drill 0.3) (layers "F.Cu" "B.Cu") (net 5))
 (via (at 56.16 36.9) (size 0.8) (drill 0.3) (layers "F.Cu" "B.Cu") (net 5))
 (segment (start 56.955 36.105) (end 56.16 36.9) (width 0.3) (layer "B.Cu") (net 5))
 (segment (start 70.56 28) (end 60.26 28) (width 0.25) (layer "B.Cu") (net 5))
 (segment (start 52.375 26.975) (end 50.8 25.4) (width 0.25) (layer "B.Cu") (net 5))
 (segment (start 60.26 28) (end 59.235 26.975) (width 0.25) (layer "B.Cu") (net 5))
 (segment (start 61.585 48.5) (end 61.585 44.6) (width 0.3) (layer "B.Cu") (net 5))
 (segment (start 62.455 36.105) (end 56.955 36.105) (width 0.3) (layer "B.Cu") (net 5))
 (segment (start 70.56 28) (end 62.455 36.105) (width 0.3) (layer "B.Cu") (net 5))
 (segment (start 59.235 26.975) (end 52.375 26.975) (width 0.25) (layer "B.Cu") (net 5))
 (segment (start 56.135 39.265) (end 56.135 40.535) (width 0.3) (layer "F.Cu") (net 6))
 (segment (start 57.817199 39.265) (end 57.817199 38.417199) (width 0.3) (layer "F.Cu") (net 6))
 (segment (start 73.015 48.5) (end 63.5 48.5) (width 0.3) (layer "F.Cu") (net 6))
 (segment (start 57.817199 38.417199) (end 57.8 38.4) (width 0.3) (layer "F.Cu") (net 6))
 (segment (start 62.682199 34.4) (end 57.817199 39.265) (width 0.3) (layer "F.Cu") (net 6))
 (segment (start 57.817199 39.265) (end 56.135 39.265) (width 0.3) (layer "F.Cu") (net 6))
 (via (at 57.8 38.4) (size 0.6) (drill 0.3) (layers "F.Cu" "B.Cu") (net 6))
 (segment (start 57.8 38.4) (end 58.75 39.35) (width 0.3) (layer "B.Cu") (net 6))
 (segment (start 58.75 39.35) (end 58.75 41.85) (width 0.3) (layer "B.Cu") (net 6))
 (segment (start 68.5123 31.9) (end 68.5123 32.0477) (width 0.2) (layer "F.Cu") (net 1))
 (segment (start 68.5123 32.0477) (end 68.3646 32.1954) (width 0.2) (layer "F.Cu") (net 1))
 (segment (start 68.636 29.4) (end 68.636 31.7763) (width 0.3) (layer "F.Cu") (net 1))
 (segment (start 68.636 31.7763) (end 68.5123 31.9) (width 0.2) (layer "F.Cu") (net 1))
 (segment (start 68.3646 32.1954) (end 68.3646 34.4) (width 0.3) (layer "F.Cu") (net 1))
 (segment (start 68.5123 29.0477) (end 68.66 28.9) (width 0.2) (layer "F.Cu") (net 1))
 (segment (start 50.210001 40.535) (end 49.760001 40.985) (width 0.3) (layer "F.Cu") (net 3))
 (segment (start 49.760001 42.100001) (end 50.115 42.455) (width 0.3) (layer "F.Cu") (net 3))
 (segment (start 71.684 33.727607) (end 65.8538 39.557807) (width 0.3) (layer "F.Cu") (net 3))
 (segment (start 61.6125 39.7062) (end 61.760893 39.557807) (width 0.3) (layer "F.Cu") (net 3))
 (segment (start 50.115 42.455) (end 58.8637 42.455) (width 0.3) (layer "F.Cu") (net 3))
 (segment (start 71.684 29.4) (end 71.684 33.727607) (width 0.3) (layer "F.Cu") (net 3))
 (segment (start 61.760893 39.557807) (end 65.8538 39.557807) (width 0.3) (layer "F.Cu") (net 3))
 (segment (start 49.760001 40.985) (end 49.760001 42.100001) (width 0.3) (layer "F.Cu") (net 3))
 (segment (start 58.8637 42.455) (end 61.6125 39.7062) (width 0.3) (layer "F.Cu") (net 3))
 (segment (start 51.185 40.535) (end 50.210001 40.535) (width 0.3) (layer "F.Cu") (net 3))
 (segment (start 55.88 26.81) (end 58.97 29.9) (width 0.3) (layer "F.Cu") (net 8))
 (segment (start 55.88 25.4) (end 55.88 26.81) (width 0.3) (layer "F.Cu") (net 8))
 (segment (start 61.8 41) (end 60.7 42.1) (width 1) (layer "F.Cu") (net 4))
 (segment (start 66.06 41) (end 61.8 41) (width 1) (layer "F.Cu") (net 4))
 (via (at 66.06 41) (size 2) (drill 0.6) (layers "F.Cu" "B.Cu") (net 4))
 (segment (start 71.76 33.3) (end 66.06 39) (width 1) (layer "B.Cu") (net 4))
 (segment (start 65.1 27) (end 70.974214 27) (width 1) (layer "B.Cu") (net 4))
 (segment (start 65.1 27) (end 63.5 25.4) (width 1) (layer "B.Cu") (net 4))
 (segment (start 66.06 39) (end 66.06 41) (width 1) (layer "B.Cu") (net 4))
 (segment (start 71.76 27.785786) (end 71.76 33.3) (width 1) (layer "B.Cu") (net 4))
 (segment (start 70.974214 27) (end 71.76 27.785786) (width 1) (layer "B.Cu") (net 4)))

